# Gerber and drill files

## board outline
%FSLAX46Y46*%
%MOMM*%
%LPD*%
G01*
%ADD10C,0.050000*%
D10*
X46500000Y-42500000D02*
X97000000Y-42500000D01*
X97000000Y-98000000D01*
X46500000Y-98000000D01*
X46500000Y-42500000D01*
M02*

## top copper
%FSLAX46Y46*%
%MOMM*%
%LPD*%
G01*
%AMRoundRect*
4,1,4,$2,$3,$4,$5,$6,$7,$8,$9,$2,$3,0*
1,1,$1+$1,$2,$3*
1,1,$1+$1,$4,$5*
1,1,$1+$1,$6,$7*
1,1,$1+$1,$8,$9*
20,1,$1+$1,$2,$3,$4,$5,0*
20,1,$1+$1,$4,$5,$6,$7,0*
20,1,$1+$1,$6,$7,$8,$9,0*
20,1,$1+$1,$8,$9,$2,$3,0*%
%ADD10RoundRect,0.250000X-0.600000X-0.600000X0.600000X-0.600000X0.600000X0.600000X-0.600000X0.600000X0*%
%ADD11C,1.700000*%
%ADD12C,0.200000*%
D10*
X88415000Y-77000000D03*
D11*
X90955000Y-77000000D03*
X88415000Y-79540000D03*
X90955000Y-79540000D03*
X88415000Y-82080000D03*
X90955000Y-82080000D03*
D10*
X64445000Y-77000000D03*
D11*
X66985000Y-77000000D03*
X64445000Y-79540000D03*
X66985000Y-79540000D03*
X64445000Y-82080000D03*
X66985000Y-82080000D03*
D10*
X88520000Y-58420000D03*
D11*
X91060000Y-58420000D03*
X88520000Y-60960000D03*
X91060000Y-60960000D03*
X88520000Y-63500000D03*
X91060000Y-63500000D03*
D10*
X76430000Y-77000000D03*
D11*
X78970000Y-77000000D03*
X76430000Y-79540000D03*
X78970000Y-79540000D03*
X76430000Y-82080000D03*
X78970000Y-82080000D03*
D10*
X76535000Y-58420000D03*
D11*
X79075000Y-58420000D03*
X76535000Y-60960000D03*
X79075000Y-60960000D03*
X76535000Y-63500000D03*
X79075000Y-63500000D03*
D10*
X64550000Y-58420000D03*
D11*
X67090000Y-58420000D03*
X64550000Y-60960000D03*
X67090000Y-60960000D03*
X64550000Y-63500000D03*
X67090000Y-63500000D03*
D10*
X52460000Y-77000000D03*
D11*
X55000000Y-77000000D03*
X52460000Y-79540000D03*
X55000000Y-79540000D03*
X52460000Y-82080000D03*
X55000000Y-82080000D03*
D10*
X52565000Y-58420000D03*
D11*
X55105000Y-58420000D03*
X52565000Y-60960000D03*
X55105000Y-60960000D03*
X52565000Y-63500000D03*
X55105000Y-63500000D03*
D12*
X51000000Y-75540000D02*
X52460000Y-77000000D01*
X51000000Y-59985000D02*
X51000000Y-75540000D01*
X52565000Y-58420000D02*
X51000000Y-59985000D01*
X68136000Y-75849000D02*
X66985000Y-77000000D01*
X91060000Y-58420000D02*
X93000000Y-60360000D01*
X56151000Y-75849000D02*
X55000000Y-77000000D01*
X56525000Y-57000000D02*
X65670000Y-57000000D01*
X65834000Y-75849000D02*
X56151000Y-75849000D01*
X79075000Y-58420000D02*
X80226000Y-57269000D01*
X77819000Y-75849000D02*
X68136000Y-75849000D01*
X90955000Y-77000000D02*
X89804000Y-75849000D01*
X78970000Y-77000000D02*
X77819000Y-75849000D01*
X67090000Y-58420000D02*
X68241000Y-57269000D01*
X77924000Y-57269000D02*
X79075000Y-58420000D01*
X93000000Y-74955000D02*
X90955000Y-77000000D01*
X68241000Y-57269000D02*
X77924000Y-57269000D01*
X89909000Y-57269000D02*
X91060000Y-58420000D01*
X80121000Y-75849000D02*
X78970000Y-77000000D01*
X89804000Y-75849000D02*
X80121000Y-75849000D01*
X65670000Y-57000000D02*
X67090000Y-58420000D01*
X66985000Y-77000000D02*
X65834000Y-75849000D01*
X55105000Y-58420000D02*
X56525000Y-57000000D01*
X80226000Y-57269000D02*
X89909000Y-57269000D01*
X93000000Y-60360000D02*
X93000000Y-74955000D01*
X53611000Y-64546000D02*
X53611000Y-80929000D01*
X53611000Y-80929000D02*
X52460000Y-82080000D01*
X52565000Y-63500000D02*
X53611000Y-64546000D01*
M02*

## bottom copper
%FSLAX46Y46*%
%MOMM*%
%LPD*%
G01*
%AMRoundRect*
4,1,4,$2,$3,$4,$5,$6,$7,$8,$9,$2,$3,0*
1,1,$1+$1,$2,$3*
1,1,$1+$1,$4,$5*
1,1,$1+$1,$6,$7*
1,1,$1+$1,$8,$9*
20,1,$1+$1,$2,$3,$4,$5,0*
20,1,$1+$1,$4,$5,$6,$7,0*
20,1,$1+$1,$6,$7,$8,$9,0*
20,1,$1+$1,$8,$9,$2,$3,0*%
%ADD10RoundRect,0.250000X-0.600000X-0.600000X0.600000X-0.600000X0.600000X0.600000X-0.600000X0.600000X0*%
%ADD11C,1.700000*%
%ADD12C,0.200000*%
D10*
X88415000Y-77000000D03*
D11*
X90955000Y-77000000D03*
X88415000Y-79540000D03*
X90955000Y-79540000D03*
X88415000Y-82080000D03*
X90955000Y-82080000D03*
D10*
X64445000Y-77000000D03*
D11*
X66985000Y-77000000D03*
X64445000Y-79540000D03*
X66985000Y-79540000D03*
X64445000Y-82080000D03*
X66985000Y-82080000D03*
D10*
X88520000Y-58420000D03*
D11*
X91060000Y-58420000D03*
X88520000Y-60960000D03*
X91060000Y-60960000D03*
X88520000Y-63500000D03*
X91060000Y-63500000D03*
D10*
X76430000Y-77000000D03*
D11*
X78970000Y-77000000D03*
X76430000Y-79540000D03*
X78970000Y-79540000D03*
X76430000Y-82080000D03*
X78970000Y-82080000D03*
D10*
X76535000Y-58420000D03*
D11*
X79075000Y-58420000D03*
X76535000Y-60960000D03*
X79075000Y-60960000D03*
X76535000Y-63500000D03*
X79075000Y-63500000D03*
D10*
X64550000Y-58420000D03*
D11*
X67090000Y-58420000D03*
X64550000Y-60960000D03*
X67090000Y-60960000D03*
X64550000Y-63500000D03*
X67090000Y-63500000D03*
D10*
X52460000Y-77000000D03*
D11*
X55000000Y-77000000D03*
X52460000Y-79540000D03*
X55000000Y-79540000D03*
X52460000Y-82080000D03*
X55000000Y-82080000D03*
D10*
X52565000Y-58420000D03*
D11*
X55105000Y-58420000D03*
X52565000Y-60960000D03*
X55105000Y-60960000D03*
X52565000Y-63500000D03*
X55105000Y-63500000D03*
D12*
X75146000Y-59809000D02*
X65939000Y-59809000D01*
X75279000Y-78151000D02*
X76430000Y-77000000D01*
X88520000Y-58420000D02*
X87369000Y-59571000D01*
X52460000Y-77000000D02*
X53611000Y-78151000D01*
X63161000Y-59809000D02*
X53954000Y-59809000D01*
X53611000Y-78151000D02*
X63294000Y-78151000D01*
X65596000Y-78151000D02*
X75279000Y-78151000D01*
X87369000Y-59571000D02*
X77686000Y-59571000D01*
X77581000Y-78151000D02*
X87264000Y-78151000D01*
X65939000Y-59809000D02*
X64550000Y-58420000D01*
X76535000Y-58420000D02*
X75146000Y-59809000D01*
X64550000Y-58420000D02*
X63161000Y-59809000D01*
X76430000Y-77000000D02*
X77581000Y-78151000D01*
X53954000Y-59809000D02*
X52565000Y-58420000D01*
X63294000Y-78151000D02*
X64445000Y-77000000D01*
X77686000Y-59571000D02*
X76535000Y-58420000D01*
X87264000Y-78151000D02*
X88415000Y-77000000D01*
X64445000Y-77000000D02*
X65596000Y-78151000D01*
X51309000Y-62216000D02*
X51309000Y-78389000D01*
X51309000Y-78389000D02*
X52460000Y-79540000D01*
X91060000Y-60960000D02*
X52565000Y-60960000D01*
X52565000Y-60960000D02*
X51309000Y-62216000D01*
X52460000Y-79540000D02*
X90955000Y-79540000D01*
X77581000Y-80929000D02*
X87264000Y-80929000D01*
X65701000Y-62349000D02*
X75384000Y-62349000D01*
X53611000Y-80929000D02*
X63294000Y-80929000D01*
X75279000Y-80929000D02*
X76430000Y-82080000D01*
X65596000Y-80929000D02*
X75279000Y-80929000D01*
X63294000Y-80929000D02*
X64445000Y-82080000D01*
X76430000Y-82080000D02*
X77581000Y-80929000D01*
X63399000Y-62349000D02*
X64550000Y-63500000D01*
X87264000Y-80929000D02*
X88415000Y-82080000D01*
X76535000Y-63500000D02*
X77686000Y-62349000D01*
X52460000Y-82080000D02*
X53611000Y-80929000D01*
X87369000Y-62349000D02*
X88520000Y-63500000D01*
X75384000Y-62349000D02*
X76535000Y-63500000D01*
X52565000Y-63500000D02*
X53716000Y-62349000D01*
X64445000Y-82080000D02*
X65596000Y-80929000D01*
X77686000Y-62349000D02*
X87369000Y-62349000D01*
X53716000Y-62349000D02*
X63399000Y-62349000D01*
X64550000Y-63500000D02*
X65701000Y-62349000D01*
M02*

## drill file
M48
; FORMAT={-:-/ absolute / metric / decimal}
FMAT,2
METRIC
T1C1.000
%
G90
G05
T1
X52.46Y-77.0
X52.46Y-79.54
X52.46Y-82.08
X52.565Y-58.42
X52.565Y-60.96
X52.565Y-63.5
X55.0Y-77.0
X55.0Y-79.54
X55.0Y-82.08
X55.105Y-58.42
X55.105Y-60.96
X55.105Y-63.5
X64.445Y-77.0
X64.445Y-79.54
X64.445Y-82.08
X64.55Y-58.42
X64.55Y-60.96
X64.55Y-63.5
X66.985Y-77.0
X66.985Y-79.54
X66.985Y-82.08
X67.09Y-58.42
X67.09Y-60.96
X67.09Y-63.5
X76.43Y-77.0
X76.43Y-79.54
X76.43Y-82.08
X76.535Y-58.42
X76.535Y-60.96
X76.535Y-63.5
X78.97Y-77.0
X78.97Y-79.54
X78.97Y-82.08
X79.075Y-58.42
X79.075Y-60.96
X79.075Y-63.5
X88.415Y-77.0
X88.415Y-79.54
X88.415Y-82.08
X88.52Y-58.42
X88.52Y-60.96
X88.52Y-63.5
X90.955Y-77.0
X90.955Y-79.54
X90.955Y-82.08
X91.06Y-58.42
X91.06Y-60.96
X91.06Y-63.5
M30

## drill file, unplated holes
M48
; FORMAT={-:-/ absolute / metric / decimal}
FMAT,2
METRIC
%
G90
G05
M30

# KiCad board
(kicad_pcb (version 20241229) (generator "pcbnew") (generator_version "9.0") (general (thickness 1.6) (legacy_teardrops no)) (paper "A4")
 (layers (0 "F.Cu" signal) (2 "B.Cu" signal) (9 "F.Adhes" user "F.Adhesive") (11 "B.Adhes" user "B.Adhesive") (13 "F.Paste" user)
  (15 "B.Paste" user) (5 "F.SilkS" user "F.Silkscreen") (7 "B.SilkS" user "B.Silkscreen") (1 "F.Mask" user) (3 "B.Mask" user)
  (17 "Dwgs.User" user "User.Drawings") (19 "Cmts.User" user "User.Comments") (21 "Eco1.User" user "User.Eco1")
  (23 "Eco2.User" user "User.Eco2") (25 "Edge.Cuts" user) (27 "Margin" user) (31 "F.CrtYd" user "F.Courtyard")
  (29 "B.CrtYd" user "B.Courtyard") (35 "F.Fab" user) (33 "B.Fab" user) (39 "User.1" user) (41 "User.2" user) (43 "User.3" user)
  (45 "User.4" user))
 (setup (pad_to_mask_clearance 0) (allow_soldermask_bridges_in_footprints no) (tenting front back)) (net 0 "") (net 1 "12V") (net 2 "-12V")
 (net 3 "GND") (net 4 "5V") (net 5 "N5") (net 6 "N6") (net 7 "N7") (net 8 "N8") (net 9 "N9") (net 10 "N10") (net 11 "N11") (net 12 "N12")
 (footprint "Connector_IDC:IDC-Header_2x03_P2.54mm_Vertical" (layer "F.Cu") (at 88.415 77)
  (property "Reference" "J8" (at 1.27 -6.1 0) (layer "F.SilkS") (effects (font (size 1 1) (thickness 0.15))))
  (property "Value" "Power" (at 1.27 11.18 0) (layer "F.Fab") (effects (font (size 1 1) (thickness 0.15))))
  (pad "1" thru_hole roundrect (at 0 0) (size 1.7 1.7) (drill 1) (layers "*.Cu" "*.Mask") (remove_unused_layers no)
   (roundrect_rratio 0.147059) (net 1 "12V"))
  (pad "2" thru_hole circle (at 2.54 0) (size 1.7 1.7) (drill 1) (layers "*.Cu" "*.Mask") (remove_unused_layers no) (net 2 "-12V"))
  (pad "3" thru_hole circle (at 0 2.54) (size 1.7 1.7) (drill 1) (layers "*.Cu" "*.Mask") (remove_unused_layers no) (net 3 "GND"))
  (pad "4" thru_hole circle (at 2.54 2.54) (size 1.7 1.7) (drill 1) (layers "*.Cu" "*.Mask") (remove_unused_layers no) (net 3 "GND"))
  (pad "5" thru_hole circle (at 0 5.08) (size 1.7 1.7) (drill 1) (layers "*.Cu" "*.Mask") (remove_unused_layers no) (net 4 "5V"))
  (pad "6" thru_hole circle (at 2.54 5.08) (size 1.7 1.7) (drill 1) (layers "*.Cu" "*.Mask") (remove_unused_layers no) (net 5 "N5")))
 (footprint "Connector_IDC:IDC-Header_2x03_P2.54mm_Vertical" (layer "F.Cu") (at 64.445 77)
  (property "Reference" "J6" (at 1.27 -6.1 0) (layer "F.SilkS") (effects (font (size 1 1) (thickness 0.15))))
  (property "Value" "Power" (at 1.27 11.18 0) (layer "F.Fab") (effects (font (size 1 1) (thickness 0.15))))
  (pad "1" thru_hole roundrect (at 0 0) (size 1.7 1.7) (drill 1) (layers "*.Cu" "*.Mask") (remove_unused_layers no)
   (roundrect_rratio 0.147059) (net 1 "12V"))
  (pad "2" thru_hole circle (at 2.54 0) (size 1.7 1.7) (drill 1) (layers "*.Cu" "*.Mask") (remove_unused_layers no) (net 2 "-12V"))
  (pad "3" thru_hole circle (at 0 2.54) (size 1.7 1.7) (drill 1) (layers "*.Cu" "*.Mask") (remove_unused_layers no) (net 3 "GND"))
  (pad "4" thru_hole circle (at 2.54 2.54) (size 1.7 1.7) (drill 1) (layers "*.Cu" "*.Mask") (remove_unused_layers no) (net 3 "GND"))
  (pad "5" thru_hole circle (at 0 5.08) (size 1.7 1.7) (drill 1) (layers "*.Cu" "*.Mask") (remove_unused_layers no) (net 4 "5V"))
  (pad "6" thru_hole circle (at 2.54 5.08) (size 1.7 1.7) (drill 1) (layers "*.Cu" "*.Mask") (remove_unused_layers no) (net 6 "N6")))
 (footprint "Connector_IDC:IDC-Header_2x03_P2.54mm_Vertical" (layer "F.Cu") (at 88.52 58.42)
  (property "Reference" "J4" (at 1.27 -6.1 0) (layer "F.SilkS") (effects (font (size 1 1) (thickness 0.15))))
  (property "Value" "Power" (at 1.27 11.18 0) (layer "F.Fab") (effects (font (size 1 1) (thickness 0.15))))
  (pad "1" thru_hole roundrect (at 0 0) (size 1.7 1.7) (drill 1) (layers "*.Cu" "*.Mask") (remove_unused_layers no)
   (roundrect_rratio 0.147059) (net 1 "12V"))
  (pad "2" thru_hole circle (at 2.54 0) (size 1.7 1.7) (drill 1) (layers "*.Cu" "*.Mask") (remove_unused_layers no) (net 2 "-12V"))
  (pad "3" thru_hole circle (at 0 2.54) (size 1.7 1.7) (drill 1) (layers "*.Cu" "*.Mask") (remove_unused_layers no) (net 3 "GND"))
  (pad "4" thru_hole circle (at 2.54 2.54) (size 1.7 1.7) (drill 1) (layers "*.Cu" "*.Mask") (remove_unused_layers no) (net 3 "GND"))
  (pad "5" thru_hole circle (at 0 5.08) (size 1.7 1.7) (drill 1) (layers "*.Cu" "*.Mask") (remove_unused_layers no) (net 4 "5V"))
  (pad "6" thru_hole circle (at 2.54 5.08) (size 1.7 1.7) (drill 1) (layers "*.Cu" "*.Mask") (remove_unused_layers no) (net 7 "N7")))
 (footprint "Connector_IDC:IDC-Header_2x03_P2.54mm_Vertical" (layer "F.Cu") (at 76.43 77)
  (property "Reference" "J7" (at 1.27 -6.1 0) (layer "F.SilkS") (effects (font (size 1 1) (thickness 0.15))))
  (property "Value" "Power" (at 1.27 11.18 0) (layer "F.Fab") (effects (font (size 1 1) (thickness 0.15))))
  (pad "1" thru_hole roundrect (at 0 0) (size 1.7 1.7) (drill 1) (layers "*.Cu" "*.Mask") (remove_unused_layers no)
   (roundrect_rratio 0.147059) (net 1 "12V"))
  (pad "2" thru_hole circle (at 2.54 0) (size 1.7 1.7) (drill 1) (layers "*.Cu" "*.Mask") (remove_unused_layers no) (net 2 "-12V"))
  (pad "3" thru_hole circle (at 0 2.54) (size 1.7 1.7) (drill 1) (layers "*.Cu" "*.Mask") (remove_unused_layers no) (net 3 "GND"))
  (pad "4" thru_hole circle (at 2.54 2.54) (size 1.7 1.7) (drill 1) (layers "*.Cu" "*.Mask") (remove_unused_layers no) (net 3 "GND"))
  (pad "5" thru_hole circle (at 0 5.08) (size 1.7 1.7) (drill 1) (layers "*.Cu" "*.Mask") (remove_unused_layers no) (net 4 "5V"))
  (pad "6" thru_hole circle (at 2.54 5.08) (size 1.7 1.7) (drill 1) (layers "*.Cu" "*.Mask") (remove_unused_layers no) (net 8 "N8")))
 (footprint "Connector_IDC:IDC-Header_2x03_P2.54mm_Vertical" (layer "F.Cu") (at 76.535 58.42)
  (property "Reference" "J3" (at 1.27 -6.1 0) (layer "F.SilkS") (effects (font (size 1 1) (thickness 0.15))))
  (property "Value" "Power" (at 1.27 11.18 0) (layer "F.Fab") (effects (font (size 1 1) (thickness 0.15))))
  (pad "1" thru_hole roundrect (at 0 0) (size 1.7 1.7) (drill 1) (layers "*.Cu" "*.Mask") (remove_unused_layers no)
   (roundrect_rratio 0.147059) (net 1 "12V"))
  (pad "2" thru_hole circle (at 2.54 0) (size 1.7 1.7) (drill 1) (layers "*.Cu" "*.Mask") (remove_unused_layers no) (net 2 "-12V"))
  (pad "3" thru_hole circle (at 0 2.54) (size 1.7 1.7) (drill 1) (layers "*.Cu" "*.Mask") (remove_unused_layers no) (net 3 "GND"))
  (pad "4" thru_hole circle (at 2.54 2.54) (size 1.7 1.7) (drill 1) (layers "*.Cu" "*.Mask") (remove_unused_layers no) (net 3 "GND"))
  (pad "5" thru_hole circle (at 0 5.08) (size 1.7 1.7) (drill 1) (layers "*.Cu" "*.Mask") (remove_unused_layers no) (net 4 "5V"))
  (pad "6" thru_hole circle (at 2.54 5.08) (size 1.7 1.7) (drill 1) (layers "*.Cu" "*.Mask") (remove_unused_layers no) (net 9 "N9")))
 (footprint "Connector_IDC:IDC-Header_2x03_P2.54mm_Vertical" (layer "F.Cu") (at 64.55 58.42)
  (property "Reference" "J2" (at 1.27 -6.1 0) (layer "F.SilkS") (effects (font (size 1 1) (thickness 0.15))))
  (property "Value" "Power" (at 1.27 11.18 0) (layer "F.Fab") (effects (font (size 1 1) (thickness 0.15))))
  (pad "1" thru_hole roundrect (at 0 0) (size 1.7 1.7) (drill 1) (layers "*.Cu" "*.Mask") (remove_unused_layers no)
   (roundrect_rratio 0.147059) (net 1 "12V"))
  (pad "2" thru_hole circle (at 2.54 0) (size 1.7 1.7) (drill 1) (layers "*.Cu" "*.Mask") (remove_unused_layers no) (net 2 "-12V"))
  (pad "3" thru_hole circle (at 0 2.54) (size 1.7 1.7) (drill 1) (layers "*.Cu" "*.Mask") (remove_unused_layers no) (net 3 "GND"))
  (pad "4" thru_hole circle (at 2.54 2.54) (size 1.7 1.7) (drill 1) (layers "*.Cu" "*.Mask") (remove_unused_layers no) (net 3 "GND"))
  (pad "5" thru_hole circle (at 0 5.08) (size 1.7 1.7) (drill 1) (layers "*.Cu" "*.Mask") (remove_unused_layers no) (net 4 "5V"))
  (pad "6" thru_hole circle (at 2.54 5.08) (size 1.7 1.7) (drill 1) (layers "*.Cu" "*.Mask") (remove_unused_layers no) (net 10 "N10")))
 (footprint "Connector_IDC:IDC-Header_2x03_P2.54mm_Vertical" (layer "F.Cu") (at 52.46 77)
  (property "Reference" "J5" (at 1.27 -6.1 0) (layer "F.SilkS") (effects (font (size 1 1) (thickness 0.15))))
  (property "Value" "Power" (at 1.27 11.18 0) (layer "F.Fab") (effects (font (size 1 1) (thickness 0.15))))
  (pad "1" thru_hole roundrect (at 0 0) (size 1.7 1.7) (drill 1) (layers "*.Cu" "*.Mask") (remove_unused_layers no)
   (roundrect_rratio 0.147059) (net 1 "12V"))
  (pad "2" thru_hole circle (at 2.54 0) (size 1.7 1.7) (drill 1) (layers "*.Cu" "*.Mask") (remove_unused_layers no) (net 2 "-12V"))
  (pad "3" thru_hole circle (at 0 2.54) (size 1.7 1.7) (drill 1) (layers "*.Cu" "*.Mask") (remove_unused_layers no) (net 3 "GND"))
  (pad "4" thru_hole circle (at 2.54 2.54) (size 1.7 1.7) (drill 1) (layers "*.Cu" "*.Mask") (remove_unused_layers no) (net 3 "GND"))
  (pad "5" thru_hole circle (at 0 5.08) (size 1.7 1.7) (drill 1) (layers "*.Cu" "*.Mask") (remove_unused_layers no) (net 4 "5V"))
  (pad "6" thru_hole circle (at 2.54 5.08) (size 1.7 1.7) (drill 1) (layers "*.Cu" "*.Mask") (remove_unused_layers no) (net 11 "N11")))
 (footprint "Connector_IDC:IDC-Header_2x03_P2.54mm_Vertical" (layer "F.Cu") (at 52.565 58.42)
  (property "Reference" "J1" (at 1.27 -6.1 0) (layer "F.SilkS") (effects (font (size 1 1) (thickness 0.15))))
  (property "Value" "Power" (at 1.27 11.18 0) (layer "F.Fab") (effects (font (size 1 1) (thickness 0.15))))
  (pad "1" thru_hole roundrect (at 0 0) (size 1.7 1.7) (drill 1) (layers "*.Cu" "*.Mask") (remove_unused_layers no)
   (roundrect_rratio 0.147059) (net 1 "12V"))
  (pad "2" thru_hole circle (at 2.54 0) (size 1.7 1.7) (drill 1) (layers "*.Cu" "*.Mask") (remove_unused_layers no) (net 2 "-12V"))
  (pad "3" thru_hole circle (at 0 2.54) (size 1.7 1.7) (drill 1) (layers "*.Cu" "*.Mask") (remove_unused_layers no) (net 3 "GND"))
  (pad "4" thru_hole circle (at 2.54 2.54) (size 1.7 1.7) (drill 1) (layers "*.Cu" "*.Mask") (remove_unused_layers no) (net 3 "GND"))
  (pad "5" thru_hole circle (at 0 5.08) (size 1.7 1.7) (drill 1) (layers "*.Cu" "*.Mask") (remove_unused_layers no) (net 4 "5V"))
  (pad "6" thru_hole circle (at 2.54 5.08) (size 1.7 1.7) (drill 1) (layers "*.Cu" "*.Mask") (remove_unused_layers no) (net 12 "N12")))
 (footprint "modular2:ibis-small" (layer "F.Cu") (at 93 93)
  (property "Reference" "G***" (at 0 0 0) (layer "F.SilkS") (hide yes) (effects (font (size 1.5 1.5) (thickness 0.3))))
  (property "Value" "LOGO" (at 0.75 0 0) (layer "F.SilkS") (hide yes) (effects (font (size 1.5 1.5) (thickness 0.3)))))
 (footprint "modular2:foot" (layer "B.Cu") (at 90 90.5 180)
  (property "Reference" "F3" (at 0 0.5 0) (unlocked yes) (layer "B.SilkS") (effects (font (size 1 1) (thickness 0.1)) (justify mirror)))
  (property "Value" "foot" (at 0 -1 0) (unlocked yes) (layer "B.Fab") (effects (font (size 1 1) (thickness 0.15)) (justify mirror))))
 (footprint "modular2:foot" (layer "B.Cu") (at 90 49.5 180)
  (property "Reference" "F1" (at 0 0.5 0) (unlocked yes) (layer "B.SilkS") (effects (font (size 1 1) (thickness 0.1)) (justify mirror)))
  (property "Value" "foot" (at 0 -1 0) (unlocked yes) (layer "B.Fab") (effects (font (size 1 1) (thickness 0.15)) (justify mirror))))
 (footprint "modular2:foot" (layer "B.Cu") (at 53.5 49.5 180)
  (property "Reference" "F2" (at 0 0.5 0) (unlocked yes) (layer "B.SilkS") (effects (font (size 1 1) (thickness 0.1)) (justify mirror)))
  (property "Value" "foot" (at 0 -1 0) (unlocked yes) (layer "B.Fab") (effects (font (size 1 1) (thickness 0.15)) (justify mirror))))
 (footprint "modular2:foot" (layer "B.Cu") (at 53.5 90.5 180)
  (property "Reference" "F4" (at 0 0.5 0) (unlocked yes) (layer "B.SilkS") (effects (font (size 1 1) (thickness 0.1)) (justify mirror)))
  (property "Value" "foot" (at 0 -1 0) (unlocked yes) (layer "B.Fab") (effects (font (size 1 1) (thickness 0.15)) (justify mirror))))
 (gr_rect (start 46.5 42.5) (end 97 98) (stroke (width 0.05) (type default)) (fill no) (layer "Edge.Cuts"))
 (segment (start 51 75.54) (end 52.46 77) (width 0.2) (layer "F.Cu") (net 1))
 (segment (start 51 59.985) (end 51 75.54) (width 0.2) (layer "F.Cu") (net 1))
 (segment (start 52.565 58.42) (end 51 59.985) (width 0.2) (layer "F.Cu") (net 1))
 (segment (start 75.146 59.809) (end 65.939 59.809) (width 0.2) (layer "B.Cu") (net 1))
 (segment (start 75.279 78.151) (end 76.43 77) (width 0.2) (layer "B.Cu") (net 1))
 (segment (start 88.52 58.42) (end 87.369 59.571) (width 0.2) (layer "B.Cu") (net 1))
 (segment (start 52.46 77) (end 53.611 78.151) (width 0.2) (layer "B.Cu") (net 1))
 (segment (start 63.161 59.809) (end 53.954 59.809) (width 0.2) (layer "B.Cu") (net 1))
 (segment (start 53.611 78.151) (end 63.294 78.151) (width 0.2) (layer "B.Cu") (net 1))
 (segment (start 65.596 78.151) (end 75.279 78.151) (width 0.2) (layer "B.Cu") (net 1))
 (segment (start 87.369 59.571) (end 77.686 59.571) (width 0.2) (layer "B.Cu") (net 1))
 (segment (start 77.581 78.151) (end 87.264 78.151) (width 0.2) (layer "B.Cu") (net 1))
 (segment (start 65.939 59.809) (end 64.55 58.42) (width 0.2) (layer "B.Cu") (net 1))
 (segment (start 76.535 58.42) (end 75.146 59.809) (width 0.2) (layer "B.Cu") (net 1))
 (segment (start 64.55 58.42) (end 63.161 59.809) (width 0.2) (layer "B.Cu") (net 1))
 (segment (start 76.43 77) (end 77.581 78.151) (width 0.2) (layer "B.Cu") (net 1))
 (segment (start 53.954 59.809) (end 52.565 58.42) (width 0.2) (layer "B.Cu") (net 1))
 (segment (start 63.294 78.151) (end 64.445 77) (width 0.2) (layer "B.Cu") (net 1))
 (segment (start 77.686 59.571) (end 76.535 58.42) (width 0.2) (layer "B.Cu") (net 1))
 (segment (start 87.264 78.151) (end 88.415 77) (width 0.2) (layer "B.Cu") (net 1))
 (segment (start 64.445 77) (end 65.596 78.151) (width 0.2) (layer "B.Cu") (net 1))
 (segment (start 51.309 62.216) (end 51.309 78.389) (width 0.2) (layer "B.Cu") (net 3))
 (segment (start 51.309 78.389) (end 52.46 79.54) (width 0.2) (layer "B.Cu") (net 3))
 (segment (start 91.06 60.96) (end 52.565 60.96) (width 0.2) (layer "B.Cu") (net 3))
 (segment (start 52.565 60.96) (end 51.309 62.216) (width 0.2) (layer "B.Cu") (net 3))
 (segment (start 52.46 79.54) (end 90.955 79.54) (width 0.2) (layer "B.Cu") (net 3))
 (segment (start 68.136 75.849) (end 66.985 77) (width 0.2) (layer "F.Cu") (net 2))
 (segment (start 91.06 58.42) (end 93 60.36) (width 0.2) (layer "F.Cu") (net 2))
 (segment (start 56.151 75.849) (end 55 77) (width 0.2) (layer "F.Cu") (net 2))
 (segment (start 56.525 57) (end 65.67 57) (width 0.2) (layer "F.Cu") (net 2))
 (segment (start 65.834 75.849) (end 56.151 75.849) (width 0.2) (layer "F.Cu") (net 2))
 (segment (start 79.075 58.42) (end 80.226 57.269) (width 0.2) (layer "F.Cu") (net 2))
 (segment (start 77.819 75.849) (end 68.136 75.849) (width 0.2) (layer "F.Cu") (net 2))
 (segment (start 90.955 77) (end 89.804 75.849) (width 0.2) (layer "F.Cu") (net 2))
 (segment (start 78.97 77) (end 77.819 75.849) (width 0.2) (layer "F.Cu") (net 2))
 (segment (start 67.09 58.42) (end 68.241 57.269) (width 0.2) (layer "F.Cu") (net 2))
 (segment (start 77.924 57.269) (end 79.075 58.42) (width 0.2) (layer "F.Cu") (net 2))
 (segment (start 93 74.955) (end 90.955 77) (width 0.2) (layer "F.Cu") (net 2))
 (segment (start 68.241 57.269) (end 77.924 57.269) (width 0.2) (layer "F.Cu") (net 2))
 (segment (start 89.909 57.269) (end 91.06 58.42) (width 0.2) (layer "F.Cu") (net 2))
 (segment (start 80.121 75.849) (end 78.97 77) (width 0.2) (layer "F.Cu") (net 2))
 (segment (start 89.804 75.849) (end 80.121 75.849) (width 0.2) (layer "F.Cu") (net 2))
 (segment (start 65.67 57) (end 67.09 58.42) (width 0.2) (layer "F.Cu") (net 2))
 (segment (start 66.985 77) (end 65.834 75.849) (width 0.2) (layer "F.Cu") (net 2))
 (segment (start 55.105 58.42) (end 56.525 57) (width 0.2) (layer "F.Cu") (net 2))
 (segment (start 80.226 57.269) (end 89.909 57.269) (width 0.2) (layer "F.Cu") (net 2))
 (segment (start 93 60.36) (end 93 74.955) (width 0.2) (layer "F.Cu") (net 2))
 (segment (start 53.611 64.546) (end 53.611 80.929) (width 0.2) (layer "F.Cu") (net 4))
 (segment (start 53.611 80.929) (end 52.46 82.08) (width 0.2) (layer "F.Cu") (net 4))
 (segment (start 52.565 63.5) (end 53.611 64.546) (width 0.2) (layer "F.Cu") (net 4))
 (segment (start 77.581 80.929) (end 87.264 80.929) (width 0.2) (layer "B.Cu") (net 4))
 (segment (start 65.701 62.349) (end 75.384 62.349) (width 0.2) (layer "B.Cu") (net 4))
 (segment (start 53.611 80.929) (end 63.294 80.929) (width 0.2) (layer "B.Cu") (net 4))
 (segment (start 75.279 80.929) (end 76.43 82.08) (width 0.2) (layer "B.Cu") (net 4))
 (segment (start 65.596 80.929) (end 75.279 80.929) (width 0.2) (layer "B.Cu") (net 4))
 (segment (start 63.294 80.929) (end 64.445 82.08) (width 0.2) (layer "B.Cu") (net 4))
 (segment (start 76.43 82.08) (end 77.581 80.929) (width 0.2) (layer "B.Cu") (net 4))
 (segment (start 63.399 62.349) (end 64.55 63.5) (width 0.2) (layer "B.Cu") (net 4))
 (segment (start 87.264 80.929) (end 88.415 82.08) (width 0.2) (layer "B.Cu") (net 4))
 (segment (start 76.535 63.5) (end 77.686 62.349) (width 0.2) (layer "B.Cu") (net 4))
 (segment (start 52.46 82.08) (end 53.611 80.929) (width 0.2) (layer "B.Cu") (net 4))
 (segment (start 87.369 62.349) (end 88.52 63.5) (width 0.2) (layer "B.Cu") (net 4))
 (segment (start 75.384 62.349) (end 76.535 63.5) (width 0.2) (layer "B.Cu") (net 4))
 (segment (start 52.565 63.5) (end 53.716 62.349) (width 0.2) (layer "B.Cu") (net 4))
 (segment (start 64.445 82.08) (end 65.596 80.929) (width 0.2) (layer "B.Cu") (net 4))
 (segment (start 77.686 62.349) (end 87.369 62.349) (width 0.2) (layer "B.Cu") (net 4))
 (segment (start 53.716 62.349) (end 63.399 62.349) (width 0.2) (layer "B.Cu") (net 4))
 (segment (start 64.55 63.5) (end 65.701 62.349) (width 0.2) (layer "B.Cu") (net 4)))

